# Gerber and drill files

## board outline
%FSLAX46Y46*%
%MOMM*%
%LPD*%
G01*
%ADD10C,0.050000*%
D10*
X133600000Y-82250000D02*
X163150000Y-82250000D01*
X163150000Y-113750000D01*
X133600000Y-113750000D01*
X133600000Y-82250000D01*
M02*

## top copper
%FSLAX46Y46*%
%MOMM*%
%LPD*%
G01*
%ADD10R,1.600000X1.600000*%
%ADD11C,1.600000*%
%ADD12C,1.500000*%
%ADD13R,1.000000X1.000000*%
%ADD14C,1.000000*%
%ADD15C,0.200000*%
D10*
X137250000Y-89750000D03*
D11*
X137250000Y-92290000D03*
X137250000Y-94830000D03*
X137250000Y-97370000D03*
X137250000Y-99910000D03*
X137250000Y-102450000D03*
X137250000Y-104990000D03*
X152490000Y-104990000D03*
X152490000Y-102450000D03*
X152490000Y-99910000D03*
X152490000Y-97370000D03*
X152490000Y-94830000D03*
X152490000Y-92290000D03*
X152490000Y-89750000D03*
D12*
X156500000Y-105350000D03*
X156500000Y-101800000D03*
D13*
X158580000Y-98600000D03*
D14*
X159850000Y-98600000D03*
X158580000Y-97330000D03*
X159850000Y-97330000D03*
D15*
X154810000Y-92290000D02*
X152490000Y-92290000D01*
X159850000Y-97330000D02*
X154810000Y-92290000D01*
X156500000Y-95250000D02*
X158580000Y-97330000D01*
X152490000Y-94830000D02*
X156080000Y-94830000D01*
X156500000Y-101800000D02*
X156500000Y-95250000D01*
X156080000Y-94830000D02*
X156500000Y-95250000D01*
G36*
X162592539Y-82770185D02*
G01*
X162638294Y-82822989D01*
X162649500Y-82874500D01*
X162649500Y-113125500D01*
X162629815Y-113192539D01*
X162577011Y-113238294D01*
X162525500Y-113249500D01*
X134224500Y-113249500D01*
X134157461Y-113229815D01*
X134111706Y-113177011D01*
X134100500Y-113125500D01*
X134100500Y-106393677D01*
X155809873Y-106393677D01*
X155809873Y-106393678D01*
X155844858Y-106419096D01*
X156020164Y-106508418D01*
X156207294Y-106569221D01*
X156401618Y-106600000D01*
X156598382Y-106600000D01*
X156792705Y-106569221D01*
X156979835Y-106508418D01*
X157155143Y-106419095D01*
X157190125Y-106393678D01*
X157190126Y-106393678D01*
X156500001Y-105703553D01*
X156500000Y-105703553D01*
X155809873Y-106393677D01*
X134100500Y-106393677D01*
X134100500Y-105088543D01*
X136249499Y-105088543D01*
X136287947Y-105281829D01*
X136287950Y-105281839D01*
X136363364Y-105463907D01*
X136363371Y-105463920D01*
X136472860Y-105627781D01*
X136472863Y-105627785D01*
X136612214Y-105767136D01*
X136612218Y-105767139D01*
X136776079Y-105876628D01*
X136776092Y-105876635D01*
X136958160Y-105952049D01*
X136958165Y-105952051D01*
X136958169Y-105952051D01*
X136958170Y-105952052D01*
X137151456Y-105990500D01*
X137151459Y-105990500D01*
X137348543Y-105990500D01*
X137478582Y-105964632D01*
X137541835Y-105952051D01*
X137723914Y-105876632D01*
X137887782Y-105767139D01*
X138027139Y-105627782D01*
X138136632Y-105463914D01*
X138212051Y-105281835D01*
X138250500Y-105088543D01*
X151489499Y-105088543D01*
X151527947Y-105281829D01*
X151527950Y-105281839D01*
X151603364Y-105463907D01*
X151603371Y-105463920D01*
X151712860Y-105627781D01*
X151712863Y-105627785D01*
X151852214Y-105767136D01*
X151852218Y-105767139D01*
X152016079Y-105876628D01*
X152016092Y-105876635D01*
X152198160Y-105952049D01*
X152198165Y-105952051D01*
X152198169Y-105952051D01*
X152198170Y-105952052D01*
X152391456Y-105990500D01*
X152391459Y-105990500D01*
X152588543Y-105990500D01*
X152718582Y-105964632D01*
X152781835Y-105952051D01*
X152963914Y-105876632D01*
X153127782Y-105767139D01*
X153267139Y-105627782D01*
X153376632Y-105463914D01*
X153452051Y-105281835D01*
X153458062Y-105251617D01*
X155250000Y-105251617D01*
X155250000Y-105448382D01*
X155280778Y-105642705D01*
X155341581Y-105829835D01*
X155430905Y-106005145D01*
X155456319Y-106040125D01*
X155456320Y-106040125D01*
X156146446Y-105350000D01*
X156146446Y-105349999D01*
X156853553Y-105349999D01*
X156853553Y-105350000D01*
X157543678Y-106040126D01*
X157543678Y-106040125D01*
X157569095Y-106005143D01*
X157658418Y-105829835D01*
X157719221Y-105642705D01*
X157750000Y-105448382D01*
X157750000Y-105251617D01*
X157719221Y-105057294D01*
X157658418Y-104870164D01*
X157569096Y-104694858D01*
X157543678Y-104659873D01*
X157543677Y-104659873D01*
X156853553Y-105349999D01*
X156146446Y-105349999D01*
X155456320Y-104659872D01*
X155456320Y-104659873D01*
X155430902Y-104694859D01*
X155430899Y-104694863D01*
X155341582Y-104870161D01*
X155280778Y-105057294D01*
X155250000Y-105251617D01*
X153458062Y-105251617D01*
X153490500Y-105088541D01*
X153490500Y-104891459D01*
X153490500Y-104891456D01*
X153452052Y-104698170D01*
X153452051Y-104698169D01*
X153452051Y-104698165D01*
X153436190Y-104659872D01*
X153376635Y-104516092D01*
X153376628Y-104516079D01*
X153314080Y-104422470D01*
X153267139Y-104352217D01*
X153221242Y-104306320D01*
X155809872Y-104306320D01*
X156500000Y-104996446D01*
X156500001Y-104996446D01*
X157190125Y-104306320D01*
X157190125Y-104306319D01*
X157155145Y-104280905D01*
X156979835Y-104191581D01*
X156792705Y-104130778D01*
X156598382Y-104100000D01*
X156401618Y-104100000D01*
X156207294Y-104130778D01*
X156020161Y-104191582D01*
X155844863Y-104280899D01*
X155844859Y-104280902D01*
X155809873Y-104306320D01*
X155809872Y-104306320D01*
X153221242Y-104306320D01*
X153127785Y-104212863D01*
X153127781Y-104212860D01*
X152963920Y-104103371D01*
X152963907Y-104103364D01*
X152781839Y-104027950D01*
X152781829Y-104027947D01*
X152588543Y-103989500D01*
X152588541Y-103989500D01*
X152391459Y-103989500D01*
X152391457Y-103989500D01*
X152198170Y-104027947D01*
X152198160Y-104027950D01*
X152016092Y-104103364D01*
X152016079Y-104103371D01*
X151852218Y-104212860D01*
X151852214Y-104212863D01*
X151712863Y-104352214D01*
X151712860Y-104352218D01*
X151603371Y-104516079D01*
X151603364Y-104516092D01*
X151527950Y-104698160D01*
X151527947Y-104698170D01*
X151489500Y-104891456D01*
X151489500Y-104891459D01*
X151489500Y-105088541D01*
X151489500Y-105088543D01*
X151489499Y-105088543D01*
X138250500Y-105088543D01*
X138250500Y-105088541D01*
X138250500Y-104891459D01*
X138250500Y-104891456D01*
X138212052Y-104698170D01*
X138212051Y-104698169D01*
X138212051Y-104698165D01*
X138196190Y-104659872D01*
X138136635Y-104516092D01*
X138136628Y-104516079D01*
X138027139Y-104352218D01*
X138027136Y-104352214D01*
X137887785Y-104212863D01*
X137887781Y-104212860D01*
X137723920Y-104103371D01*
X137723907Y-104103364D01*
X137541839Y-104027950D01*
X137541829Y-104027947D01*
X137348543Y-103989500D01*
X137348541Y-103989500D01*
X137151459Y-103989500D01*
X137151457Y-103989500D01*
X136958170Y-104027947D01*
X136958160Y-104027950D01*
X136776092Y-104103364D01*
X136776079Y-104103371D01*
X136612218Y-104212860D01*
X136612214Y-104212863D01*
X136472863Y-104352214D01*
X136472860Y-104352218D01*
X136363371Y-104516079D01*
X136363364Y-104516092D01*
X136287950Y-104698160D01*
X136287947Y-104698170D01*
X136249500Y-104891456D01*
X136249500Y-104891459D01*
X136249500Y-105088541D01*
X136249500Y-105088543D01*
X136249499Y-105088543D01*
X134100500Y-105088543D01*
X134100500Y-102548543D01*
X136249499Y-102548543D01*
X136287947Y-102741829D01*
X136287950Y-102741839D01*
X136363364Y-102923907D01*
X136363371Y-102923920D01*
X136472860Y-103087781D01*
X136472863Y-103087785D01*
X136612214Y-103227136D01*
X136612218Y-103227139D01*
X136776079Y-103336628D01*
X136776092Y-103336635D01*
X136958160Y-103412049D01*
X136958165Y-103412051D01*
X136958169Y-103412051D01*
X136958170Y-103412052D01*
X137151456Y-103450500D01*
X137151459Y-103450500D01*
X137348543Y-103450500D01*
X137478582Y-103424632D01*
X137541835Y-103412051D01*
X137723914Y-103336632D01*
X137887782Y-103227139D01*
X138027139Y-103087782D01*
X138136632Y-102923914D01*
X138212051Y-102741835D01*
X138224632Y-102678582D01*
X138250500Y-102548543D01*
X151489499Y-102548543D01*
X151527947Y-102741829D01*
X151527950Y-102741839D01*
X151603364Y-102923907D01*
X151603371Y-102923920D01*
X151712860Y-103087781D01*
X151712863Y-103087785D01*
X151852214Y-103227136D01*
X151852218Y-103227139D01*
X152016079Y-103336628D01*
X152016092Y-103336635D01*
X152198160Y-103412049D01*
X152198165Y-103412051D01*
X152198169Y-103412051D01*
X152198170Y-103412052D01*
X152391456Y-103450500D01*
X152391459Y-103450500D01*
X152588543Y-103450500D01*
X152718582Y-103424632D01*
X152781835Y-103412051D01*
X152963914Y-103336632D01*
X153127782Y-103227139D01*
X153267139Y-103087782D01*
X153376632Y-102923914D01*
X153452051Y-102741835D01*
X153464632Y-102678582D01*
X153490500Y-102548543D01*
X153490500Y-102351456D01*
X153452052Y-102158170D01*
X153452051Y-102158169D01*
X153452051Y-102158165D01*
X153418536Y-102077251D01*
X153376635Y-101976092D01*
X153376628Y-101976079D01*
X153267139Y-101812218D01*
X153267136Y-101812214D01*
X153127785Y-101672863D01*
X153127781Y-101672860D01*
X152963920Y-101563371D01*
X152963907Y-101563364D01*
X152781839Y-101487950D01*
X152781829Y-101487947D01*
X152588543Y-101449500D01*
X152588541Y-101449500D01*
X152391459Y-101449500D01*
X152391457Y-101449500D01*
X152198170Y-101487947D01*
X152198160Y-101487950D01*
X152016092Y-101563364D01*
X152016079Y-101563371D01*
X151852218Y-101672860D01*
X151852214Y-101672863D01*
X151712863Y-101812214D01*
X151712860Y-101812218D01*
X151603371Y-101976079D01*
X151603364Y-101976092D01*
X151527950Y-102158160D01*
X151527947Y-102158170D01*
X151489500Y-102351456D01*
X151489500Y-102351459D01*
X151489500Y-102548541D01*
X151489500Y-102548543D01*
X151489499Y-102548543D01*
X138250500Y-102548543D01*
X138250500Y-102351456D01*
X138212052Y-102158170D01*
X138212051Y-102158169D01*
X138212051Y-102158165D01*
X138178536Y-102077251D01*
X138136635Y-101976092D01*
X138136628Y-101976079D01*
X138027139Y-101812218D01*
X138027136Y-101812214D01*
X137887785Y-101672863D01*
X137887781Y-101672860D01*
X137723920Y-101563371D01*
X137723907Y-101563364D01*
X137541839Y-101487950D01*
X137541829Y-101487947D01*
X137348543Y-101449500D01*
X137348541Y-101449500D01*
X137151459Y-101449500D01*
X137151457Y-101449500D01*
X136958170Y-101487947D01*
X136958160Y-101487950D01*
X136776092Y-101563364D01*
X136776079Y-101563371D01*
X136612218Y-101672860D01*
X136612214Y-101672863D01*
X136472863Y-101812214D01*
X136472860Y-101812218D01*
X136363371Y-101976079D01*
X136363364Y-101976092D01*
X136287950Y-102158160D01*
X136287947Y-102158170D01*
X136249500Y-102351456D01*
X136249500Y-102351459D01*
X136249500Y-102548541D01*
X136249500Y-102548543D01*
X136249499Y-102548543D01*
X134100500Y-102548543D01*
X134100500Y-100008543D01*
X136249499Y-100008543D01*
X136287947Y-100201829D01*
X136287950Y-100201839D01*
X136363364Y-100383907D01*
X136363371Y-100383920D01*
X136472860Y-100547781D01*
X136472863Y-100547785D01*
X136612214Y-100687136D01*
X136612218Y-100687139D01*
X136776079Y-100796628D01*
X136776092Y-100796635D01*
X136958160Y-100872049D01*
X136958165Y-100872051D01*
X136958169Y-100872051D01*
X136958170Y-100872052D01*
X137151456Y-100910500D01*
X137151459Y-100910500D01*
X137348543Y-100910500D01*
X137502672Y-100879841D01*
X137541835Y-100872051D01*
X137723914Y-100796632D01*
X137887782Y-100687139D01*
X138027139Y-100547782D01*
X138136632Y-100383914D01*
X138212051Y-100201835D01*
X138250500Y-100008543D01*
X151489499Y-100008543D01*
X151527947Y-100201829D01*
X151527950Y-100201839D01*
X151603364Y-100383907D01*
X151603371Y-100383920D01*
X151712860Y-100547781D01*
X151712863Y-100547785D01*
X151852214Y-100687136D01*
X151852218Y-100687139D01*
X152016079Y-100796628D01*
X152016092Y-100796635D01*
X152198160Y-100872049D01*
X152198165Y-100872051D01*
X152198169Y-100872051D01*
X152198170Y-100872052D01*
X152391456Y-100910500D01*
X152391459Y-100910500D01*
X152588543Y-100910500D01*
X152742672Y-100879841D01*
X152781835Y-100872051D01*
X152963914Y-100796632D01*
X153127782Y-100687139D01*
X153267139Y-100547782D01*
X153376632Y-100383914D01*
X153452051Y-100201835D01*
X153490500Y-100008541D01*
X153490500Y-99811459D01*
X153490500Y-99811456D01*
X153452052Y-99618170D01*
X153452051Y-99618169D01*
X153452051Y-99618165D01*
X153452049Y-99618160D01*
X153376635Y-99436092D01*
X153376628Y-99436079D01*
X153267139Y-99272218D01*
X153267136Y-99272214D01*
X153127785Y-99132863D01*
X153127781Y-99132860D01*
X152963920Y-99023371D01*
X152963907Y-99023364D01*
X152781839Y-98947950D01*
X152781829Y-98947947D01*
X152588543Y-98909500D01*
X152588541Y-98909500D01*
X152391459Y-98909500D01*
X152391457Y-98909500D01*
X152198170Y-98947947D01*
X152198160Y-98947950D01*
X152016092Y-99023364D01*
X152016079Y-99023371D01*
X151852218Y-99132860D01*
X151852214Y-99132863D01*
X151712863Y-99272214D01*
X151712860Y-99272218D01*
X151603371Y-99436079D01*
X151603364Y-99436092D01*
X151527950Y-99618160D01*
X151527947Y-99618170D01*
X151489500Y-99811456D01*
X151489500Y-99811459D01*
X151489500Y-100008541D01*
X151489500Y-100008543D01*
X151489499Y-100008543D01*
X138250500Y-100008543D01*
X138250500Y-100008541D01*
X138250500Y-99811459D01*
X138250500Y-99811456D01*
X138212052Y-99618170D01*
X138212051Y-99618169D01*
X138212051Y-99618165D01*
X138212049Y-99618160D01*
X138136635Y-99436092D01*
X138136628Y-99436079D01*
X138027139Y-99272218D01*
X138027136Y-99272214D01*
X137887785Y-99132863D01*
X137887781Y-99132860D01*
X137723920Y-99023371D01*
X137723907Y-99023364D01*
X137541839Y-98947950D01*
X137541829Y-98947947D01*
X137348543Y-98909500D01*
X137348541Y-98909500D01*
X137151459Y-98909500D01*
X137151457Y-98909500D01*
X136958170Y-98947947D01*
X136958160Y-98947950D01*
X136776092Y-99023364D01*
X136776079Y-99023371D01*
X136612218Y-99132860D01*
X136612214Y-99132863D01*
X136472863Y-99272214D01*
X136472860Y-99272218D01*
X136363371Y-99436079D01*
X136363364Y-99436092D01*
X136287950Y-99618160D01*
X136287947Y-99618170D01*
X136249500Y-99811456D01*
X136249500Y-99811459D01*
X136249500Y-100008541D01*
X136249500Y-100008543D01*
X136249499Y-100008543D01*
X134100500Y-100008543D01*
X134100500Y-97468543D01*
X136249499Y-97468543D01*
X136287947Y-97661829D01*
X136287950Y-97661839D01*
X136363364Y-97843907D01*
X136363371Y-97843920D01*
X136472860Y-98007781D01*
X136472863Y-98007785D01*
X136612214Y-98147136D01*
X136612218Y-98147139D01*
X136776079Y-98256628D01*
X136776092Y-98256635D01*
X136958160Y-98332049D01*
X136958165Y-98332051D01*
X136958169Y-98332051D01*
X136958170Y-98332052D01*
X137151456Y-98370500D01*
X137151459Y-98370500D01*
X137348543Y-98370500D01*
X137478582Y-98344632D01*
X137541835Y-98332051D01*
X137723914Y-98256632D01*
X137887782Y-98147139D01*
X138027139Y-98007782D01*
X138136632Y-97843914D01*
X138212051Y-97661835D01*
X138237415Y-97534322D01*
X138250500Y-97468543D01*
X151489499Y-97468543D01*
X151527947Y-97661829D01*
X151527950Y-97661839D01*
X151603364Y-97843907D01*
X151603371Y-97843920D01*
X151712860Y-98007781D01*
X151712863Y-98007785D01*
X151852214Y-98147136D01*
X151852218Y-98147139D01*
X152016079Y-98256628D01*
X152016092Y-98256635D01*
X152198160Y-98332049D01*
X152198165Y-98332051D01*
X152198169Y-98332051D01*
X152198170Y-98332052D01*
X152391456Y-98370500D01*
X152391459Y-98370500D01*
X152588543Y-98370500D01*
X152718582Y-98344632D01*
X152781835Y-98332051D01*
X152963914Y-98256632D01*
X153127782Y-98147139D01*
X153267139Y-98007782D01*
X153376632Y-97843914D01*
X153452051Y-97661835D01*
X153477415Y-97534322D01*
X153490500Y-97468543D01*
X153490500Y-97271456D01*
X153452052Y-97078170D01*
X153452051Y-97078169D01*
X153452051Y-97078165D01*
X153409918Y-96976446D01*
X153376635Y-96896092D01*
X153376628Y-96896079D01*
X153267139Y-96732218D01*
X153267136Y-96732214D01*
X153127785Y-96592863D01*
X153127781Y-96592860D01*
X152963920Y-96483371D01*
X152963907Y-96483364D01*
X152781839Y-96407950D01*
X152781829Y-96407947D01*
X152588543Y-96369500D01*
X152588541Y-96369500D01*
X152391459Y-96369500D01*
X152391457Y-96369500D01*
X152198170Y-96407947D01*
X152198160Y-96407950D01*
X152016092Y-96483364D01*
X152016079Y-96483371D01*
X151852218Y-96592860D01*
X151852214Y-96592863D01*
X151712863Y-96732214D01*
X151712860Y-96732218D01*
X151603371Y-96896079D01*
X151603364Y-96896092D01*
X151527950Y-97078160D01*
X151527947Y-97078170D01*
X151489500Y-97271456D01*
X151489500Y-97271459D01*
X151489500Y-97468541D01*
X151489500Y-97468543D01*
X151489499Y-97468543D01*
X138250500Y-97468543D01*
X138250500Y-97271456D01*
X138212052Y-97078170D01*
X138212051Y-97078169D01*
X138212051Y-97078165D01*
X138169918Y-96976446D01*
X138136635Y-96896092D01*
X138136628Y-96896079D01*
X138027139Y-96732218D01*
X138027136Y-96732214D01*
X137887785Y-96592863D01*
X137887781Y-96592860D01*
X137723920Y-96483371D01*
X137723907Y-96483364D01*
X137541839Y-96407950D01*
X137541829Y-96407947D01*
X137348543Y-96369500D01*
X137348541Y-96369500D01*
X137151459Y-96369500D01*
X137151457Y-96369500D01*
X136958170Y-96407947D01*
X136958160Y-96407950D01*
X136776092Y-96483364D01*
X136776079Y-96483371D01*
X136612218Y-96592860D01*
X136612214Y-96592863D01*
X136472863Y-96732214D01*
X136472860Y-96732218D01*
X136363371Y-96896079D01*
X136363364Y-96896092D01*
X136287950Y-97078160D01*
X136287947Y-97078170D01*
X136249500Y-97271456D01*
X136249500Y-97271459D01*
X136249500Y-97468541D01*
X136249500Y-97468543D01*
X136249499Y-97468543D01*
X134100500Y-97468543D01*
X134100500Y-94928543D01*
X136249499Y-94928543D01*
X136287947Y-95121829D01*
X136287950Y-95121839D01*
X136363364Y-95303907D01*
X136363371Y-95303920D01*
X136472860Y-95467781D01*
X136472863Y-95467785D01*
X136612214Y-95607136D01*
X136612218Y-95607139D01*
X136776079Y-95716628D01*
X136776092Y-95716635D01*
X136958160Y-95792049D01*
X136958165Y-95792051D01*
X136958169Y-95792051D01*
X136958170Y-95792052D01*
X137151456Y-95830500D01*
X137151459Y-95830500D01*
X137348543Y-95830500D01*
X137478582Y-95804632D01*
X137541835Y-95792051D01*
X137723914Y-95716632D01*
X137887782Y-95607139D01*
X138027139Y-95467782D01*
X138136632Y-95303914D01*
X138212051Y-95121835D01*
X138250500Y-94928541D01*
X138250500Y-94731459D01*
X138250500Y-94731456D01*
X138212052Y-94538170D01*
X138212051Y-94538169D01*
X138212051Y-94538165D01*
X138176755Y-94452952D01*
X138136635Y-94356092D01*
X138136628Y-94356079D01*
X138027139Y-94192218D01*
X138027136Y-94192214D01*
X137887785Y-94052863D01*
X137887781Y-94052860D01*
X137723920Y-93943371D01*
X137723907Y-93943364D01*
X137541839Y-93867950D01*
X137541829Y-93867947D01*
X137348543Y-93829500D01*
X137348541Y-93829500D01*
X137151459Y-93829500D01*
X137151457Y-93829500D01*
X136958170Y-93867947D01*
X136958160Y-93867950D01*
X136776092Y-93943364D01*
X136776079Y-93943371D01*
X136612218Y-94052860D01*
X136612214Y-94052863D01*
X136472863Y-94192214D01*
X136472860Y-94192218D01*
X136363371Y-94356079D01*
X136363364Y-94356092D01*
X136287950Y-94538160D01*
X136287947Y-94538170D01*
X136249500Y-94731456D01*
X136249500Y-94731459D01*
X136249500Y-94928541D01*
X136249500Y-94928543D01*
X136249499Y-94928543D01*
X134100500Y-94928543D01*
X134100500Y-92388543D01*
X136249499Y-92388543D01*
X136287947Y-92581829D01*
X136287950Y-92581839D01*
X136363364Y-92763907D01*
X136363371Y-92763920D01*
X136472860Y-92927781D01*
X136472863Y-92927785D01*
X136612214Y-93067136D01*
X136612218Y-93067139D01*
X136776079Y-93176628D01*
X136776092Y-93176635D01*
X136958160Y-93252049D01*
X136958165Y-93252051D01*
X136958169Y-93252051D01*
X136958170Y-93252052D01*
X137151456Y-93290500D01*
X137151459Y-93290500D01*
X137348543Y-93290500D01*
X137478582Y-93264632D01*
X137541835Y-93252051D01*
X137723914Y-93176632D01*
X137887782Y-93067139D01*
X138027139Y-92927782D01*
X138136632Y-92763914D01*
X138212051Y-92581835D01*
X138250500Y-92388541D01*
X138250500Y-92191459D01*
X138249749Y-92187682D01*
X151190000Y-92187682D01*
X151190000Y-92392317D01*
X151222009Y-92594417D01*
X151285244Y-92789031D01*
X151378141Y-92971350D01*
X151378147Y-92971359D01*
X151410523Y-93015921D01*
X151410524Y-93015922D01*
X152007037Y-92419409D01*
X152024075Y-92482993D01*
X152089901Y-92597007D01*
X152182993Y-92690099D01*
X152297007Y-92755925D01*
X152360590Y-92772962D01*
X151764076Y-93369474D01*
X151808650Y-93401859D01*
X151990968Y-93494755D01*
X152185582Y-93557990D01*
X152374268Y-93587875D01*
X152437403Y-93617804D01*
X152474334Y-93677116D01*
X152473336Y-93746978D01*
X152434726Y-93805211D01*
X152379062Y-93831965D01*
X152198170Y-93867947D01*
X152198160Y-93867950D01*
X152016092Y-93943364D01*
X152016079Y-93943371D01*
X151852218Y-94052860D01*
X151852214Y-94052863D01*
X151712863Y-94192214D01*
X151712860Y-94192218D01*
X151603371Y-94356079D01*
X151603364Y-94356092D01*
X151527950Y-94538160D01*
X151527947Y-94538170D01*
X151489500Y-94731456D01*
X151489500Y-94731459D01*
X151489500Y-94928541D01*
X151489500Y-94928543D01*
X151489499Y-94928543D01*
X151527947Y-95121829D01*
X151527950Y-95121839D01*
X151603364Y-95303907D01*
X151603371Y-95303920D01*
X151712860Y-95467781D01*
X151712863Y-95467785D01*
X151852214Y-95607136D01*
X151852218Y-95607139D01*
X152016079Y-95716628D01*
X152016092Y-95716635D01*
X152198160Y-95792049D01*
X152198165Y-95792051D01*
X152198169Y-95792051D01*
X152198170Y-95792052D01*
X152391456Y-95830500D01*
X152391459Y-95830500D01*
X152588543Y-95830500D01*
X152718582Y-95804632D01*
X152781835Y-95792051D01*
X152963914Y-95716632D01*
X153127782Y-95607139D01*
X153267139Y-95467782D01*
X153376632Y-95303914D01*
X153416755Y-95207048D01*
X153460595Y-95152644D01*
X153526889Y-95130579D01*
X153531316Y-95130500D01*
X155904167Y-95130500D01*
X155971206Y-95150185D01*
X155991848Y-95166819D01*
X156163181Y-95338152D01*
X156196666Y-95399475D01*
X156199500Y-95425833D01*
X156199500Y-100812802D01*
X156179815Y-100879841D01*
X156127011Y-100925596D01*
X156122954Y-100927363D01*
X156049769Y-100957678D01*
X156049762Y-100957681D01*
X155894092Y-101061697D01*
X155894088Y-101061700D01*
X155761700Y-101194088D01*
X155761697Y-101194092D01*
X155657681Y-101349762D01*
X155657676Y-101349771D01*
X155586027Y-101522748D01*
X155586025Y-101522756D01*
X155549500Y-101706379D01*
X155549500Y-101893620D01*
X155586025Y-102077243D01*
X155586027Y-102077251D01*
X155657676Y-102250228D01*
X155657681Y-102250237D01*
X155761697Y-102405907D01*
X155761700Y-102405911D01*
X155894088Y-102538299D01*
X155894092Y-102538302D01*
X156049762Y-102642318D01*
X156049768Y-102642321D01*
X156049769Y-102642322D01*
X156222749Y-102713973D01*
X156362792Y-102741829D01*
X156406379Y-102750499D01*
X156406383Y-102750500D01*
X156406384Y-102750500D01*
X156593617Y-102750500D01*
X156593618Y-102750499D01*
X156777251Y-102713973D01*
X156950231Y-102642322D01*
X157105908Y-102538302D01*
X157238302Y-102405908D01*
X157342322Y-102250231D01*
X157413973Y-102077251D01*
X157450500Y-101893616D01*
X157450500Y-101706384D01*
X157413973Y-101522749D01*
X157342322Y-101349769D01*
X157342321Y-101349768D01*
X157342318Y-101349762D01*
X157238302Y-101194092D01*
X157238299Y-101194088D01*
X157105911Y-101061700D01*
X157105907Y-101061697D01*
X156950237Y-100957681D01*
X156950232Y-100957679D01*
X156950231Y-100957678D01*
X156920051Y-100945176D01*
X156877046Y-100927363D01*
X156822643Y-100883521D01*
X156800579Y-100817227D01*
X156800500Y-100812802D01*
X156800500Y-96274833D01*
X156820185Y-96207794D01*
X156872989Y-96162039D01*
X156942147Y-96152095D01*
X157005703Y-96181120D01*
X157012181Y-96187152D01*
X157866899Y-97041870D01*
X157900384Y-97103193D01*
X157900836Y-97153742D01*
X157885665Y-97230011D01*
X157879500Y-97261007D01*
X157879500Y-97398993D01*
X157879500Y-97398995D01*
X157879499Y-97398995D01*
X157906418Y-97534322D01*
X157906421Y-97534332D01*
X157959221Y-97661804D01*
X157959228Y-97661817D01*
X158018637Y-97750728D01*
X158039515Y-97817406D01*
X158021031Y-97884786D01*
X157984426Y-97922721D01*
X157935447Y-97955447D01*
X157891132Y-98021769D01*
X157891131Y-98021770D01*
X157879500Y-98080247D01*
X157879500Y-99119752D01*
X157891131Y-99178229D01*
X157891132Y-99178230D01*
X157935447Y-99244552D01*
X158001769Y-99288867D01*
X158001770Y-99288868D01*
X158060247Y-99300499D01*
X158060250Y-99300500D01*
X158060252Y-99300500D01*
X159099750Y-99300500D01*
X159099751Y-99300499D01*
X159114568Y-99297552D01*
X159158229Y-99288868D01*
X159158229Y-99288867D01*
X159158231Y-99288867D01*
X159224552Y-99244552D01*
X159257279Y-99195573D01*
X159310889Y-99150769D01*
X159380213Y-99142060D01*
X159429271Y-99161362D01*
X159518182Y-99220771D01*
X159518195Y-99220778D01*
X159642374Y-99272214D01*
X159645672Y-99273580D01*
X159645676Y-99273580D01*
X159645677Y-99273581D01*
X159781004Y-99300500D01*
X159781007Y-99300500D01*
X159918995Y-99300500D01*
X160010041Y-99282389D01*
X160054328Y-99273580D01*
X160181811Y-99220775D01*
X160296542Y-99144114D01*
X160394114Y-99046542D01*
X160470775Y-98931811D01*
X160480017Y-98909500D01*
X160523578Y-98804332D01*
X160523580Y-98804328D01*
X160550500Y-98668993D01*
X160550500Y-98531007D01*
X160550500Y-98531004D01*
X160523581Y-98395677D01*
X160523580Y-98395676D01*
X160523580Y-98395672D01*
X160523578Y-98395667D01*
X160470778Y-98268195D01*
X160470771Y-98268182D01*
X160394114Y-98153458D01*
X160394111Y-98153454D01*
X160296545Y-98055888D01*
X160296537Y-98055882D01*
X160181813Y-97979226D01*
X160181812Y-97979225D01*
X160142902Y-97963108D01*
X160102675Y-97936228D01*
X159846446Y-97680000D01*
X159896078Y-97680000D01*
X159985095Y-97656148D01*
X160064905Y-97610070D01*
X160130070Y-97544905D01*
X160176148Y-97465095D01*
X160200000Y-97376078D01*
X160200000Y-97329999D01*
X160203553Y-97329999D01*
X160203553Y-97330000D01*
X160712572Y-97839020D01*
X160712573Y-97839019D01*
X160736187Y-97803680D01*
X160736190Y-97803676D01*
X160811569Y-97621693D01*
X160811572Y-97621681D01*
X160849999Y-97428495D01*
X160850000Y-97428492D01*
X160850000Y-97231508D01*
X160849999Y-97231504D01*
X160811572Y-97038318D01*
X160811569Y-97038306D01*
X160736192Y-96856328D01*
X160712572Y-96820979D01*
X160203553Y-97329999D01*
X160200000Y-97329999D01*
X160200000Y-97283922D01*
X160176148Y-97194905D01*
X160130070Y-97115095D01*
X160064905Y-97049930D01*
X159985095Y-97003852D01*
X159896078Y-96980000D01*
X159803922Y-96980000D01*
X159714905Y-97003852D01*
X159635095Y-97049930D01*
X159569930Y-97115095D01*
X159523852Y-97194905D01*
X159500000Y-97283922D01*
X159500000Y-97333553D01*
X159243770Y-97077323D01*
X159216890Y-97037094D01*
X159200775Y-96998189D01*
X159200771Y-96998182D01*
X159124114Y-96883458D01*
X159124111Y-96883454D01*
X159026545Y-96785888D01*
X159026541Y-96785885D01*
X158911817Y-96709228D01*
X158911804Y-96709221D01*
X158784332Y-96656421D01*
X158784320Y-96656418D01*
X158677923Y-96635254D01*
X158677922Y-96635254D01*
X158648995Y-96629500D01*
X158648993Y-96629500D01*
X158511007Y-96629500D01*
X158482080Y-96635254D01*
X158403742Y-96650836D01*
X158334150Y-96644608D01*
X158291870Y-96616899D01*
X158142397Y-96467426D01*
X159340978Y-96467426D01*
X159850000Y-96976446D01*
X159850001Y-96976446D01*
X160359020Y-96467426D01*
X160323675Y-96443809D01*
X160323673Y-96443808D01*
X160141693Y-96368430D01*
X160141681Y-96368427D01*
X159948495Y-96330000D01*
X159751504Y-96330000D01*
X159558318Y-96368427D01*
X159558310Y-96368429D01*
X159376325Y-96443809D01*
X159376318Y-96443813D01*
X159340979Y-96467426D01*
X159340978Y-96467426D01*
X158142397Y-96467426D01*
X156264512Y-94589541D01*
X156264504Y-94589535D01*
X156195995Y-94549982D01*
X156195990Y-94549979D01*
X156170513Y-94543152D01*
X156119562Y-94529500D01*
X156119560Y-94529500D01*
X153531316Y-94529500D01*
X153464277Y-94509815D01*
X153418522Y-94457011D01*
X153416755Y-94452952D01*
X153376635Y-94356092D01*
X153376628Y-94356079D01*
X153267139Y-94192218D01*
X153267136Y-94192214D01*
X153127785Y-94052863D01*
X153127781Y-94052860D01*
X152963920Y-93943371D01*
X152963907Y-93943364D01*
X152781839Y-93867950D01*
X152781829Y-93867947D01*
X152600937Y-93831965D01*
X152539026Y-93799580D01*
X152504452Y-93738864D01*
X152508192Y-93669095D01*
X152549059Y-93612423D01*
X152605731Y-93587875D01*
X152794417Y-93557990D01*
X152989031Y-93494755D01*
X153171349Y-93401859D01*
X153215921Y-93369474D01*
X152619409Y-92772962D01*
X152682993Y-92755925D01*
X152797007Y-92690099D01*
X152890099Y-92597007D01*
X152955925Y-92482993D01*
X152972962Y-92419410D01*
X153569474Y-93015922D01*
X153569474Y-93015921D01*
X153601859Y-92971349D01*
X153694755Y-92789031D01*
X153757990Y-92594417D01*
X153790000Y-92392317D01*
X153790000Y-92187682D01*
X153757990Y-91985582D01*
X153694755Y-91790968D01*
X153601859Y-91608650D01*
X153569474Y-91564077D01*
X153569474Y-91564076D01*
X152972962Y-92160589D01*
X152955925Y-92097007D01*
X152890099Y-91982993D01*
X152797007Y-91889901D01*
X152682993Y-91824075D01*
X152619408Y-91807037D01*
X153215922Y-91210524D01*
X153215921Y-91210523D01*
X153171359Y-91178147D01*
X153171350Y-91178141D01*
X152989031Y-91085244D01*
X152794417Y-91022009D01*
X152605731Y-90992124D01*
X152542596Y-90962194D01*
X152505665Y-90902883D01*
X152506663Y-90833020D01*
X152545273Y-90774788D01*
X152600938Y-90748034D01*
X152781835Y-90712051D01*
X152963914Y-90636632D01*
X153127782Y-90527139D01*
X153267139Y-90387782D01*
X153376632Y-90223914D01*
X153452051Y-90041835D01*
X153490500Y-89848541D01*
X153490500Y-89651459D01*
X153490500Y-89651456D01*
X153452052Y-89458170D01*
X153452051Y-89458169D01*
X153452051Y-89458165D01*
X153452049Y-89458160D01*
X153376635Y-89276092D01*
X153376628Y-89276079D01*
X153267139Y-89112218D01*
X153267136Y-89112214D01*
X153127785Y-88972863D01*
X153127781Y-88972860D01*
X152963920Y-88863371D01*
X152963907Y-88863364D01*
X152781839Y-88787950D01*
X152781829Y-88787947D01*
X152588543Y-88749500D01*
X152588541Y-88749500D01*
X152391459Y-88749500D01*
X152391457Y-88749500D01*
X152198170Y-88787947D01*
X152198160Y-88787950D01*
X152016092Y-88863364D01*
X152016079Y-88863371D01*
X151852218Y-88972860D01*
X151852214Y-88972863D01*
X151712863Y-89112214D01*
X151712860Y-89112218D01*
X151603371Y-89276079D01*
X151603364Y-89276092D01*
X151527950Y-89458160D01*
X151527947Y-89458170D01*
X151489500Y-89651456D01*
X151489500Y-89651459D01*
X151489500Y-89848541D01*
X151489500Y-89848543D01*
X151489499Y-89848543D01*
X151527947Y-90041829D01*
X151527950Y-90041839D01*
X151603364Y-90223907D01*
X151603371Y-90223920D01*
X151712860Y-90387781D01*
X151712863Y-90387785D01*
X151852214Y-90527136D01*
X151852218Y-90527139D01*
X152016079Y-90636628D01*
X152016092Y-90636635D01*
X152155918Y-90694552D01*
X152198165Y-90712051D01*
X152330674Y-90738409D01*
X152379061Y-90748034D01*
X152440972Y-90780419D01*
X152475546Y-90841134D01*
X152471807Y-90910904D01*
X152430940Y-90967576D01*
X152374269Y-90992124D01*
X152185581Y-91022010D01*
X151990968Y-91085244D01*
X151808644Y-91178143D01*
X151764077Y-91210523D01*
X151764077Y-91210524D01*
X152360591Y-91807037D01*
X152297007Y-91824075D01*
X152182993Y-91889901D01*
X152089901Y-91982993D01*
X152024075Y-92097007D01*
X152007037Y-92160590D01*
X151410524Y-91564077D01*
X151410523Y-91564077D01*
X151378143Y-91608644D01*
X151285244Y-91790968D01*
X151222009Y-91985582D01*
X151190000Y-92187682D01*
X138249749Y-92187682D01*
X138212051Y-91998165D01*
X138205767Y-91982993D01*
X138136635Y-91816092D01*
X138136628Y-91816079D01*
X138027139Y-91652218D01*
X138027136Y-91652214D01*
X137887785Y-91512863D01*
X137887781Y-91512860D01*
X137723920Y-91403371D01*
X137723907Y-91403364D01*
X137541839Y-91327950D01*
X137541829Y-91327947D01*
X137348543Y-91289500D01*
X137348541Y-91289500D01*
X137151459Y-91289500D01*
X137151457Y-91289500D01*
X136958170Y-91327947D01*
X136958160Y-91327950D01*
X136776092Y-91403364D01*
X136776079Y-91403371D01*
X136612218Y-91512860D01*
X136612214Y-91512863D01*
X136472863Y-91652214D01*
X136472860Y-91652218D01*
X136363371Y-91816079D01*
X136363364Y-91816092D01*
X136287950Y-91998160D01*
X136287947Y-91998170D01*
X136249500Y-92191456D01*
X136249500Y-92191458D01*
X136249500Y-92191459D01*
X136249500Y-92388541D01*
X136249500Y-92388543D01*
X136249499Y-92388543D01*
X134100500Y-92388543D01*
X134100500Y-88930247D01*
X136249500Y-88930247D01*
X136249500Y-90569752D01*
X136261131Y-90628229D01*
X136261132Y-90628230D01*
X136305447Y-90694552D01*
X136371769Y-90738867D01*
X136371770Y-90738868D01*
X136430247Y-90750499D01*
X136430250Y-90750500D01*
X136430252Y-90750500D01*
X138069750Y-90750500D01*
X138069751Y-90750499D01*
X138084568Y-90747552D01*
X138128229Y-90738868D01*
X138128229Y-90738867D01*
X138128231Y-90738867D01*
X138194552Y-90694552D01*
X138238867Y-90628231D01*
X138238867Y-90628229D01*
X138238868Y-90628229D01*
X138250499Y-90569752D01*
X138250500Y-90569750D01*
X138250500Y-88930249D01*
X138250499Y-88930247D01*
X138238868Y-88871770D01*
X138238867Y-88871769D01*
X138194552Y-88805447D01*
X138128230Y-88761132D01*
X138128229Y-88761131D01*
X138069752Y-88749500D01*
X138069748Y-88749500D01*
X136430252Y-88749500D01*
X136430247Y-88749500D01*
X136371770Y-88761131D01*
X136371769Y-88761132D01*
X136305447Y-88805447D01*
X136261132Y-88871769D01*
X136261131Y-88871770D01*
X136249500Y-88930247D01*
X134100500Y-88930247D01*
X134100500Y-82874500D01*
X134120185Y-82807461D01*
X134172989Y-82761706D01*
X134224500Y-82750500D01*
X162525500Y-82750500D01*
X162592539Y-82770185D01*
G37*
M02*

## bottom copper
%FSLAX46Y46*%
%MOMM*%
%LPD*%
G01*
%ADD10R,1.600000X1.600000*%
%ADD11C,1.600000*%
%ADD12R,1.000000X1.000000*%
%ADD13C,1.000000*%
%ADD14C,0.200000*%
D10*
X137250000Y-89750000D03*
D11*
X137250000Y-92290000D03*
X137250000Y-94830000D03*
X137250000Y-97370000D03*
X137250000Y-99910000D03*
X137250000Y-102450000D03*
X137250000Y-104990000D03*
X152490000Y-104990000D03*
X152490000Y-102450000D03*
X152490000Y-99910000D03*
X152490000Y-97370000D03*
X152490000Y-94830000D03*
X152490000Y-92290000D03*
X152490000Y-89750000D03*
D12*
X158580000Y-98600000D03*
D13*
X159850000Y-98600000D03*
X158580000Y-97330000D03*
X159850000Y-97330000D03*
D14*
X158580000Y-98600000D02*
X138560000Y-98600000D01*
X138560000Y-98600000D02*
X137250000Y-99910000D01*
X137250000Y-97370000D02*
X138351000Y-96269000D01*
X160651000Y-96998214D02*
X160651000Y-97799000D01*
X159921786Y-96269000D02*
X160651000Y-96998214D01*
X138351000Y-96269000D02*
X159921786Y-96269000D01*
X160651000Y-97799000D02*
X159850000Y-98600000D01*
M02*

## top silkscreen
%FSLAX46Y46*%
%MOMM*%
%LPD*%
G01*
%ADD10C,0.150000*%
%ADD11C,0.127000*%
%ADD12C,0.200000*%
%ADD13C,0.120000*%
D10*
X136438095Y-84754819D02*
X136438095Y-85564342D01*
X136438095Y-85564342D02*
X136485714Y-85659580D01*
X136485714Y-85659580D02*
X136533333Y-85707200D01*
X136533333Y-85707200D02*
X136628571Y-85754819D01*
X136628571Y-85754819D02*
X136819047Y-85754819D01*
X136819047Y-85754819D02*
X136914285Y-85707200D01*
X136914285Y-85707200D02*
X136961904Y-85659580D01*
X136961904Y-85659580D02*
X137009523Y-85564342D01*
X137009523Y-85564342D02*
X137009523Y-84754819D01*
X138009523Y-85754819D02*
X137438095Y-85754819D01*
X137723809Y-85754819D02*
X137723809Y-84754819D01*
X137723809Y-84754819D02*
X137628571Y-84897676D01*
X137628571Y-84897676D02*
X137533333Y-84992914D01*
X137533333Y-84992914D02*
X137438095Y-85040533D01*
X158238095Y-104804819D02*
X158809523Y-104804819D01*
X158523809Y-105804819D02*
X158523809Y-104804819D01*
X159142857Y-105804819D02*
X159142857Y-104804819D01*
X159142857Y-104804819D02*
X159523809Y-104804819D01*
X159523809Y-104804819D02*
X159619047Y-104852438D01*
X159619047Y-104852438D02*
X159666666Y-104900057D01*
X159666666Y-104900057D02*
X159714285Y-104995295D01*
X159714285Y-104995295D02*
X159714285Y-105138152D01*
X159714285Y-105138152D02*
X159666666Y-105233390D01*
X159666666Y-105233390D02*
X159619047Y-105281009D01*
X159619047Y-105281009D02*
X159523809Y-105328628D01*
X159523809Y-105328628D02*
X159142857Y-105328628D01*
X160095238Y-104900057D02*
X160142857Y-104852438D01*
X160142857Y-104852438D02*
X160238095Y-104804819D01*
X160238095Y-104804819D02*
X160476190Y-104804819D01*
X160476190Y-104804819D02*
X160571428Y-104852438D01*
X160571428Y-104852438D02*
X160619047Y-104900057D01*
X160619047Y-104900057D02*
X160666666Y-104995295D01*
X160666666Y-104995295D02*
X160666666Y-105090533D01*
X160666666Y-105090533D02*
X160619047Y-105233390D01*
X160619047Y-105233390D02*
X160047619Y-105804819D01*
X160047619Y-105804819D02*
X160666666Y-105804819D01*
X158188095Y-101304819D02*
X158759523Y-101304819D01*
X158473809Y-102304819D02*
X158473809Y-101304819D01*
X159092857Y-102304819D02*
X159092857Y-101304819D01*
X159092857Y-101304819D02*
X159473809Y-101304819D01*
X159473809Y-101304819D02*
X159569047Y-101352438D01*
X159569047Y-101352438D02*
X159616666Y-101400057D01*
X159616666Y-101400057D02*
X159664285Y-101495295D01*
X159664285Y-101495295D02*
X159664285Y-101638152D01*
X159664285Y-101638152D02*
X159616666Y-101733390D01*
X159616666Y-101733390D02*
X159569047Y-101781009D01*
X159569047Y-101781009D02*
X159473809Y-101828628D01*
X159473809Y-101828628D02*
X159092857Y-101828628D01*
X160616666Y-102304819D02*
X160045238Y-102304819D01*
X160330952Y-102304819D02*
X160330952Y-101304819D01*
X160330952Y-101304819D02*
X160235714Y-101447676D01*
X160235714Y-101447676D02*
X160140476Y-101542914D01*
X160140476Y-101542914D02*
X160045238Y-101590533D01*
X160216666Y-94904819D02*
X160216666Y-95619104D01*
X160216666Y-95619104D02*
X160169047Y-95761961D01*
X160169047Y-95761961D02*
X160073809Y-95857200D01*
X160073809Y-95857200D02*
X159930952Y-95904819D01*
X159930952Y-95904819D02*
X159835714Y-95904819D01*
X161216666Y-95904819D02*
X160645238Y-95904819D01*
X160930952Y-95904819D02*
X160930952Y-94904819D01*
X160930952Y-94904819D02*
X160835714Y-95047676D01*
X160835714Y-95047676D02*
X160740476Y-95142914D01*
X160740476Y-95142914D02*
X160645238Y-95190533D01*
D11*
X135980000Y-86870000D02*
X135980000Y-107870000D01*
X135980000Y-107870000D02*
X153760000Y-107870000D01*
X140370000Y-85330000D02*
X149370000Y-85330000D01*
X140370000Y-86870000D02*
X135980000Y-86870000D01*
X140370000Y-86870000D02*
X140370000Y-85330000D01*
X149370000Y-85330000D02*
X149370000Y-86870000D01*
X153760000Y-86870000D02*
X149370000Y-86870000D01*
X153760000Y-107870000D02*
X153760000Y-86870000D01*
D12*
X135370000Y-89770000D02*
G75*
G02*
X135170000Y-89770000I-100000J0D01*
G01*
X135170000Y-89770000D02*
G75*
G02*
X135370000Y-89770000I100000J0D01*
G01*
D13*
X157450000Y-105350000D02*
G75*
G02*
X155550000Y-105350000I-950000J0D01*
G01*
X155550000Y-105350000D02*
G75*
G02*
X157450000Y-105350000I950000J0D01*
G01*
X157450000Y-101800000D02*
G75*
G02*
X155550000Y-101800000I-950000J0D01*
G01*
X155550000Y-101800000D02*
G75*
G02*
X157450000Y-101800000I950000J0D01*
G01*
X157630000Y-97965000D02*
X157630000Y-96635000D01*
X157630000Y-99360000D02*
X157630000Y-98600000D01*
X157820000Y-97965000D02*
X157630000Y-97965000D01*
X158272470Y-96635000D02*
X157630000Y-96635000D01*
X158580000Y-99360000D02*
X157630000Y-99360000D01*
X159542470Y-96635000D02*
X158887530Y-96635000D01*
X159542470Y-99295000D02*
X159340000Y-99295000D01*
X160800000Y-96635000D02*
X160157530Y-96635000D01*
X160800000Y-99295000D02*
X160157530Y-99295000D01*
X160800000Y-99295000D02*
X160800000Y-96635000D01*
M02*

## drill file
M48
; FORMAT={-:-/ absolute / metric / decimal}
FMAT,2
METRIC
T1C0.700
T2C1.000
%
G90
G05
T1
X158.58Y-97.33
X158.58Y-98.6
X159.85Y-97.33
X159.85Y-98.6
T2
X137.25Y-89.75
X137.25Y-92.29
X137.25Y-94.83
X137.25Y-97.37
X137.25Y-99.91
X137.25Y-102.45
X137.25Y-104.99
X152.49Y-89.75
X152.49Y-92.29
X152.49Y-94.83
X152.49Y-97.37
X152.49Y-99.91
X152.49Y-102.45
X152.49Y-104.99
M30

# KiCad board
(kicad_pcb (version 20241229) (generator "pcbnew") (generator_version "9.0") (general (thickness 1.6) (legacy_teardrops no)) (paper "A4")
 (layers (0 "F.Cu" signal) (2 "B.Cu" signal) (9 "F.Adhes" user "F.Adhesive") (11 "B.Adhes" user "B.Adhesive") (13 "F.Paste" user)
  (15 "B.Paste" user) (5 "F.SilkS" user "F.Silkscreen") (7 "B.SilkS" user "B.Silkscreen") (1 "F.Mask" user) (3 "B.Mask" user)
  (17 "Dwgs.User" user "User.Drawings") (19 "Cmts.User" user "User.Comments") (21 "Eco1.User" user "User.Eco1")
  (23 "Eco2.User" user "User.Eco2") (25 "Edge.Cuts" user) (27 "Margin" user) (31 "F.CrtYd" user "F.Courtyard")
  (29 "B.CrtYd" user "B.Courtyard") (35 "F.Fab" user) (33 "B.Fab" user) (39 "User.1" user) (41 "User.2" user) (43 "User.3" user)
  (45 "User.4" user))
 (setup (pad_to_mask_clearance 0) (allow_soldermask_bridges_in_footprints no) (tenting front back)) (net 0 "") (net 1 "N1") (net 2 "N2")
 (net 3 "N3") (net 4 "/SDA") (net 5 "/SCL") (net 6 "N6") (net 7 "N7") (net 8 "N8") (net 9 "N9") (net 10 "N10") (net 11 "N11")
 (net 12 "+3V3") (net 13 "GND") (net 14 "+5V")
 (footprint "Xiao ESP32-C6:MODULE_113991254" (layer "F.Cu") (at 144.87 97.37)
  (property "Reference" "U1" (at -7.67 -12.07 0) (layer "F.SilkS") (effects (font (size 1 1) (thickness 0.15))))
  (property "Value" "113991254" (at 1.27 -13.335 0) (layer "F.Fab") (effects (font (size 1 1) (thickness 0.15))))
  (fp_line (start -8.89 -10.5) (end -8.89 10.5) (stroke (width 0.127) (type solid)) (layer "F.SilkS"))
  (fp_line (start -8.89 10.5) (end 8.89 10.5) (stroke (width 0.127) (type solid)) (layer "F.SilkS"))
  (fp_line (start -4.5 -12.04) (end 4.5 -12.04) (stroke (width 0.127) (type solid)) (layer "F.SilkS"))
  (fp_line (start -4.5 -10.5) (end -8.89 -10.5) (stroke (width 0.127) (type solid)) (layer "F.SilkS"))
  (fp_line (start -4.5 -10.5) (end -4.5 -12.04) (stroke (width 0.127) (type solid)) (layer "F.SilkS"))
  (fp_line (start 4.5 -12.04) (end 4.5 -10.5) (stroke (width 0.127) (type solid)) (layer "F.SilkS"))
  (fp_line (start 8.89 -10.5) (end 4.5 -10.5) (stroke (width 0.127) (type solid)) (layer "F.SilkS"))
  (fp_line (start 8.89 10.5) (end 8.89 -10.5) (stroke (width 0.127) (type solid)) (layer "F.SilkS"))
  (fp_circle (center -9.6 -7.6) (end -9.5 -7.6) (stroke (width 0.2) (type solid)) (fill no) (layer "F.SilkS"))
  (pad "1" thru_hole rect (at -7.62 -7.62) (size 1.6 1.6) (drill 1) (layers "*.Cu" "*.Mask") (remove_unused_layers no) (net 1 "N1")
   (solder_mask_margin 0.102))
  (pad "2" thru_hole circle (at -7.62 -5.08) (size 1.6 1.6) (drill 1) (layers "*.Cu" "*.Mask") (remove_unused_layers no) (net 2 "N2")
   (solder_mask_margin 0.102))
  (pad "3" thru_hole circle (at -7.62 -2.54) (size 1.6 1.6) (drill 1) (layers "*.Cu" "*.Mask") (remove_unused_layers no) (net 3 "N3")
   (solder_mask_margin 0.102))
  (pad "4" thru_hole circle (at -7.62 0) (size 1.6 1.6) (drill 1) (layers "*.Cu" "*.Mask") (remove_unused_layers no) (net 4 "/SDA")
   (solder_mask_margin 0.102))
  (pad "5" thru_hole circle (at -7.62 2.54) (size 1.6 1.6) (drill 1) (layers "*.Cu" "*.Mask") (remove_unused_layers no) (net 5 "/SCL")
   (solder_mask_margin 0.102))
  (pad "6" thru_hole circle (at -7.62 5.08) (size 1.6 1.6) (drill 1) (layers "*.Cu" "*.Mask") (remove_unused_layers no) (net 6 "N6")
   (solder_mask_margin 0.102))
  (pad "7" thru_hole circle (at -7.62 7.62) (size 1.6 1.6) (drill 1) (layers "*.Cu" "*.Mask") (remove_unused_layers no) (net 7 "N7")
   (solder_mask_margin 0.102))
  (pad "8" thru_hole circle (at 7.62 7.62) (size 1.6 1.6) (drill 1) (layers "*.Cu" "*.Mask") (remove_unused_layers no) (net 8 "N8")
   (solder_mask_margin 0.102))
  (pad "9" thru_hole circle (at 7.62 5.08) (size 1.6 1.6) (drill 1) (layers "*.Cu" "*.Mask") (remove_unused_layers no) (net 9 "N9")
   (solder_mask_margin 0.102))
  (pad "10" thru_hole circle (at 7.62 2.54) (size 1.6 1.6) (drill 1) (layers "*.Cu" "*.Mask") (remove_unused_layers no) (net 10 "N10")
   (solder_mask_margin 0.102))
  (pad "11" thru_hole circle (at 7.62 0) (size 1.6 1.6) (drill 1) (layers "*.Cu" "*.Mask") (remove_unused_layers no) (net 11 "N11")
   (solder_mask_margin 0.102))
  (pad "12" thru_hole circle (at 7.62 -2.54) (size 1.6 1.6) (drill 1) (layers "*.Cu" "*.Mask") (remove_unused_layers no) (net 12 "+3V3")
   (solder_mask_margin 0.102))
  (pad "13" thru_hole circle (at 7.62 -5.08) (size 1.6 1.6) (drill 1) (layers "*.Cu" "*.Mask") (remove_unused_layers no) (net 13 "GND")
   (solder_mask_margin 0.102))
  (pad "14" thru_hole circle (at 7.62 -7.62) (size 1.6 1.6) (drill 1) (layers "*.Cu" "*.Mask") (remove_unused_layers no) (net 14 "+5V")
   (solder_mask_margin 0.102)))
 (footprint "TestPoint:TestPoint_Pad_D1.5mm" (layer "F.Cu") (at 156.5 105.35)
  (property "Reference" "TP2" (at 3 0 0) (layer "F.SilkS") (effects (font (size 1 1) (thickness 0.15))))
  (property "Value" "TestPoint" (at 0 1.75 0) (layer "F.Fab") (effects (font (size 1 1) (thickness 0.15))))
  (fp_circle (center 0 0) (end 0 0.95) (stroke (width 0.12) (type solid)) (fill no) (layer "F.SilkS"))
  (pad "1" smd circle (at 0 0) (size 1.5 1.5) (layers "F.Cu" "F.Mask") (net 13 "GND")))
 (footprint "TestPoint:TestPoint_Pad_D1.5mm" (layer "F.Cu") (at 156.5 101.8)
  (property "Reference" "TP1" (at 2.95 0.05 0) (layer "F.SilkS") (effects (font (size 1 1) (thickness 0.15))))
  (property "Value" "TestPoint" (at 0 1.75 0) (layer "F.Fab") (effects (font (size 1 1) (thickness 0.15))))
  (fp_circle (center 0 0) (end 0 0.95) (stroke (width 0.12) (type solid)) (fill no) (layer "F.SilkS"))
  (pad "1" smd circle (at 0 0) (size 1.5 1.5) (layers "F.Cu" "F.Mask") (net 12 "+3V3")))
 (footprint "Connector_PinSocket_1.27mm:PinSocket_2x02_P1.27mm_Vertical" (layer "F.Cu") (at 158.58 98.6 180)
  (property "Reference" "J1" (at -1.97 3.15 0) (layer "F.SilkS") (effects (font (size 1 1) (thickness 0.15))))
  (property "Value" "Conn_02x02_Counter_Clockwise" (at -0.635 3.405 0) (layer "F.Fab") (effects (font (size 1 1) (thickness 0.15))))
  (fp_line (start 0.95 0.635) (end 0.95 1.965) (stroke (width 0.12) (type solid)) (layer "F.SilkS"))
  (fp_line (start 0.95 -0.76) (end 0.95 0) (stroke (width 0.12) (type solid)) (layer "F.SilkS"))
  (fp_line (start 0.76 0.635) (end 0.95 0.635) (stroke (width 0.12) (type solid)) (layer "F.SilkS"))
  (fp_line (start 0.30753 1.965) (end 0.95 1.965) (stroke (width 0.12) (type solid)) (layer "F.SilkS"))
  (fp_line (start 0 -0.76) (end 0.95 -0.76) (stroke (width 0.12) (type solid)) (layer "F.SilkS"))
  (fp_line (start -0.96247 1.965) (end -0.30753 1.965) (stroke (width 0.12) (type solid)) (layer "F.SilkS"))
  (fp_line (start -0.96247 -0.695) (end -0.76 -0.695) (stroke (width 0.12) (type solid)) (layer "F.SilkS"))
  (fp_line (start -2.22 1.965) (end -1.57753 1.965) (stroke (width 0.12) (type solid)) (layer "F.SilkS"))
  (fp_line (start -2.22 -0.695) (end -1.57753 -0.695) (stroke (width 0.12) (type solid)) (layer "F.SilkS"))
  (fp_line (start -2.22 -0.695) (end -2.22 1.965) (stroke (width 0.12) (type solid)) (layer "F.SilkS"))
  (pad "1" thru_hole rect (at 0 0 180) (size 1 1) (drill 0.7) (layers "*.Cu" "*.Mask") (remove_unused_layers no) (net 5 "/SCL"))
  (pad "2" thru_hole circle (at -1.27 0 180) (size 1 1) (drill 0.7) (layers "*.Cu" "*.Mask") (remove_unused_layers no) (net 4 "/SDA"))
  (pad "3" thru_hole circle (at 0 1.27 180) (size 1 1) (drill 0.7) (layers "*.Cu" "*.Mask") (remove_unused_layers no) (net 12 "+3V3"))
  (pad "4" thru_hole circle (at -1.27 1.27 180) (size 1 1) (drill 0.7) (layers "*.Cu" "*.Mask") (remove_unused_layers no) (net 13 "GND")))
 (gr_rect (start 133.6 82.25) (end 163.15 113.75) (stroke (width 0.05) (type default)) (fill no) (layer "Edge.Cuts"))
 (segment (start 158.58 98.6) (end 138.56 98.6) (width 0.2) (layer "B.Cu") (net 5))
 (segment (start 138.56 98.6) (end 137.25 99.91) (width 0.2) (layer "B.Cu") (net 5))
 (segment (start 137.25 97.37) (end 138.351 96.269) (width 0.2) (layer "B.Cu") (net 4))
 (segment (start 160.651 96.998214) (end 160.651 97.799) (width 0.2) (layer "B.Cu") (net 4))
 (segment (start 159.921786 96.269) (end 160.651 96.998214) (width 0.2) (layer "B.Cu") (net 4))
 (segment (start 138.351 96.269) (end 159.921786 96.269) (width 0.2) (layer "B.Cu") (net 4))
 (segment (start 160.651 97.799) (end 159.85 98.6) (width 0.2) (layer "B.Cu") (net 4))
 (segment (start 154.81 92.29) (end 152.49 92.29) (width 0.2) (layer "F.Cu") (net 13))
 (segment (start 159.85 97.33) (end 154.81 92.29) (width 0.2) (layer "F.Cu") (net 13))
 (segment (start 156.5 95.25) (end 158.58 97.33) (width 0.2) (layer "F.Cu") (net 12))
 (segment (start 152.49 94.83) (end 156.08 94.83) (width 0.2) (layer "F.Cu") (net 12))
 (segment (start 156.5 101.8) (end 156.5 95.25) (width 0.2) (layer "F.Cu") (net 12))
 (segment (start 156.08 94.83) (end 156.5 95.25) (width 0.2) (layer "F.Cu") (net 12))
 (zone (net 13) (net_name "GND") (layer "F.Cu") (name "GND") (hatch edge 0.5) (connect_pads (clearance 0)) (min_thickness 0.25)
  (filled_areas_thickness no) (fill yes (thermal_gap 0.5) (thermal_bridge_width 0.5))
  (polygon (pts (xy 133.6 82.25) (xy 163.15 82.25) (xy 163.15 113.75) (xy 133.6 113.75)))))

